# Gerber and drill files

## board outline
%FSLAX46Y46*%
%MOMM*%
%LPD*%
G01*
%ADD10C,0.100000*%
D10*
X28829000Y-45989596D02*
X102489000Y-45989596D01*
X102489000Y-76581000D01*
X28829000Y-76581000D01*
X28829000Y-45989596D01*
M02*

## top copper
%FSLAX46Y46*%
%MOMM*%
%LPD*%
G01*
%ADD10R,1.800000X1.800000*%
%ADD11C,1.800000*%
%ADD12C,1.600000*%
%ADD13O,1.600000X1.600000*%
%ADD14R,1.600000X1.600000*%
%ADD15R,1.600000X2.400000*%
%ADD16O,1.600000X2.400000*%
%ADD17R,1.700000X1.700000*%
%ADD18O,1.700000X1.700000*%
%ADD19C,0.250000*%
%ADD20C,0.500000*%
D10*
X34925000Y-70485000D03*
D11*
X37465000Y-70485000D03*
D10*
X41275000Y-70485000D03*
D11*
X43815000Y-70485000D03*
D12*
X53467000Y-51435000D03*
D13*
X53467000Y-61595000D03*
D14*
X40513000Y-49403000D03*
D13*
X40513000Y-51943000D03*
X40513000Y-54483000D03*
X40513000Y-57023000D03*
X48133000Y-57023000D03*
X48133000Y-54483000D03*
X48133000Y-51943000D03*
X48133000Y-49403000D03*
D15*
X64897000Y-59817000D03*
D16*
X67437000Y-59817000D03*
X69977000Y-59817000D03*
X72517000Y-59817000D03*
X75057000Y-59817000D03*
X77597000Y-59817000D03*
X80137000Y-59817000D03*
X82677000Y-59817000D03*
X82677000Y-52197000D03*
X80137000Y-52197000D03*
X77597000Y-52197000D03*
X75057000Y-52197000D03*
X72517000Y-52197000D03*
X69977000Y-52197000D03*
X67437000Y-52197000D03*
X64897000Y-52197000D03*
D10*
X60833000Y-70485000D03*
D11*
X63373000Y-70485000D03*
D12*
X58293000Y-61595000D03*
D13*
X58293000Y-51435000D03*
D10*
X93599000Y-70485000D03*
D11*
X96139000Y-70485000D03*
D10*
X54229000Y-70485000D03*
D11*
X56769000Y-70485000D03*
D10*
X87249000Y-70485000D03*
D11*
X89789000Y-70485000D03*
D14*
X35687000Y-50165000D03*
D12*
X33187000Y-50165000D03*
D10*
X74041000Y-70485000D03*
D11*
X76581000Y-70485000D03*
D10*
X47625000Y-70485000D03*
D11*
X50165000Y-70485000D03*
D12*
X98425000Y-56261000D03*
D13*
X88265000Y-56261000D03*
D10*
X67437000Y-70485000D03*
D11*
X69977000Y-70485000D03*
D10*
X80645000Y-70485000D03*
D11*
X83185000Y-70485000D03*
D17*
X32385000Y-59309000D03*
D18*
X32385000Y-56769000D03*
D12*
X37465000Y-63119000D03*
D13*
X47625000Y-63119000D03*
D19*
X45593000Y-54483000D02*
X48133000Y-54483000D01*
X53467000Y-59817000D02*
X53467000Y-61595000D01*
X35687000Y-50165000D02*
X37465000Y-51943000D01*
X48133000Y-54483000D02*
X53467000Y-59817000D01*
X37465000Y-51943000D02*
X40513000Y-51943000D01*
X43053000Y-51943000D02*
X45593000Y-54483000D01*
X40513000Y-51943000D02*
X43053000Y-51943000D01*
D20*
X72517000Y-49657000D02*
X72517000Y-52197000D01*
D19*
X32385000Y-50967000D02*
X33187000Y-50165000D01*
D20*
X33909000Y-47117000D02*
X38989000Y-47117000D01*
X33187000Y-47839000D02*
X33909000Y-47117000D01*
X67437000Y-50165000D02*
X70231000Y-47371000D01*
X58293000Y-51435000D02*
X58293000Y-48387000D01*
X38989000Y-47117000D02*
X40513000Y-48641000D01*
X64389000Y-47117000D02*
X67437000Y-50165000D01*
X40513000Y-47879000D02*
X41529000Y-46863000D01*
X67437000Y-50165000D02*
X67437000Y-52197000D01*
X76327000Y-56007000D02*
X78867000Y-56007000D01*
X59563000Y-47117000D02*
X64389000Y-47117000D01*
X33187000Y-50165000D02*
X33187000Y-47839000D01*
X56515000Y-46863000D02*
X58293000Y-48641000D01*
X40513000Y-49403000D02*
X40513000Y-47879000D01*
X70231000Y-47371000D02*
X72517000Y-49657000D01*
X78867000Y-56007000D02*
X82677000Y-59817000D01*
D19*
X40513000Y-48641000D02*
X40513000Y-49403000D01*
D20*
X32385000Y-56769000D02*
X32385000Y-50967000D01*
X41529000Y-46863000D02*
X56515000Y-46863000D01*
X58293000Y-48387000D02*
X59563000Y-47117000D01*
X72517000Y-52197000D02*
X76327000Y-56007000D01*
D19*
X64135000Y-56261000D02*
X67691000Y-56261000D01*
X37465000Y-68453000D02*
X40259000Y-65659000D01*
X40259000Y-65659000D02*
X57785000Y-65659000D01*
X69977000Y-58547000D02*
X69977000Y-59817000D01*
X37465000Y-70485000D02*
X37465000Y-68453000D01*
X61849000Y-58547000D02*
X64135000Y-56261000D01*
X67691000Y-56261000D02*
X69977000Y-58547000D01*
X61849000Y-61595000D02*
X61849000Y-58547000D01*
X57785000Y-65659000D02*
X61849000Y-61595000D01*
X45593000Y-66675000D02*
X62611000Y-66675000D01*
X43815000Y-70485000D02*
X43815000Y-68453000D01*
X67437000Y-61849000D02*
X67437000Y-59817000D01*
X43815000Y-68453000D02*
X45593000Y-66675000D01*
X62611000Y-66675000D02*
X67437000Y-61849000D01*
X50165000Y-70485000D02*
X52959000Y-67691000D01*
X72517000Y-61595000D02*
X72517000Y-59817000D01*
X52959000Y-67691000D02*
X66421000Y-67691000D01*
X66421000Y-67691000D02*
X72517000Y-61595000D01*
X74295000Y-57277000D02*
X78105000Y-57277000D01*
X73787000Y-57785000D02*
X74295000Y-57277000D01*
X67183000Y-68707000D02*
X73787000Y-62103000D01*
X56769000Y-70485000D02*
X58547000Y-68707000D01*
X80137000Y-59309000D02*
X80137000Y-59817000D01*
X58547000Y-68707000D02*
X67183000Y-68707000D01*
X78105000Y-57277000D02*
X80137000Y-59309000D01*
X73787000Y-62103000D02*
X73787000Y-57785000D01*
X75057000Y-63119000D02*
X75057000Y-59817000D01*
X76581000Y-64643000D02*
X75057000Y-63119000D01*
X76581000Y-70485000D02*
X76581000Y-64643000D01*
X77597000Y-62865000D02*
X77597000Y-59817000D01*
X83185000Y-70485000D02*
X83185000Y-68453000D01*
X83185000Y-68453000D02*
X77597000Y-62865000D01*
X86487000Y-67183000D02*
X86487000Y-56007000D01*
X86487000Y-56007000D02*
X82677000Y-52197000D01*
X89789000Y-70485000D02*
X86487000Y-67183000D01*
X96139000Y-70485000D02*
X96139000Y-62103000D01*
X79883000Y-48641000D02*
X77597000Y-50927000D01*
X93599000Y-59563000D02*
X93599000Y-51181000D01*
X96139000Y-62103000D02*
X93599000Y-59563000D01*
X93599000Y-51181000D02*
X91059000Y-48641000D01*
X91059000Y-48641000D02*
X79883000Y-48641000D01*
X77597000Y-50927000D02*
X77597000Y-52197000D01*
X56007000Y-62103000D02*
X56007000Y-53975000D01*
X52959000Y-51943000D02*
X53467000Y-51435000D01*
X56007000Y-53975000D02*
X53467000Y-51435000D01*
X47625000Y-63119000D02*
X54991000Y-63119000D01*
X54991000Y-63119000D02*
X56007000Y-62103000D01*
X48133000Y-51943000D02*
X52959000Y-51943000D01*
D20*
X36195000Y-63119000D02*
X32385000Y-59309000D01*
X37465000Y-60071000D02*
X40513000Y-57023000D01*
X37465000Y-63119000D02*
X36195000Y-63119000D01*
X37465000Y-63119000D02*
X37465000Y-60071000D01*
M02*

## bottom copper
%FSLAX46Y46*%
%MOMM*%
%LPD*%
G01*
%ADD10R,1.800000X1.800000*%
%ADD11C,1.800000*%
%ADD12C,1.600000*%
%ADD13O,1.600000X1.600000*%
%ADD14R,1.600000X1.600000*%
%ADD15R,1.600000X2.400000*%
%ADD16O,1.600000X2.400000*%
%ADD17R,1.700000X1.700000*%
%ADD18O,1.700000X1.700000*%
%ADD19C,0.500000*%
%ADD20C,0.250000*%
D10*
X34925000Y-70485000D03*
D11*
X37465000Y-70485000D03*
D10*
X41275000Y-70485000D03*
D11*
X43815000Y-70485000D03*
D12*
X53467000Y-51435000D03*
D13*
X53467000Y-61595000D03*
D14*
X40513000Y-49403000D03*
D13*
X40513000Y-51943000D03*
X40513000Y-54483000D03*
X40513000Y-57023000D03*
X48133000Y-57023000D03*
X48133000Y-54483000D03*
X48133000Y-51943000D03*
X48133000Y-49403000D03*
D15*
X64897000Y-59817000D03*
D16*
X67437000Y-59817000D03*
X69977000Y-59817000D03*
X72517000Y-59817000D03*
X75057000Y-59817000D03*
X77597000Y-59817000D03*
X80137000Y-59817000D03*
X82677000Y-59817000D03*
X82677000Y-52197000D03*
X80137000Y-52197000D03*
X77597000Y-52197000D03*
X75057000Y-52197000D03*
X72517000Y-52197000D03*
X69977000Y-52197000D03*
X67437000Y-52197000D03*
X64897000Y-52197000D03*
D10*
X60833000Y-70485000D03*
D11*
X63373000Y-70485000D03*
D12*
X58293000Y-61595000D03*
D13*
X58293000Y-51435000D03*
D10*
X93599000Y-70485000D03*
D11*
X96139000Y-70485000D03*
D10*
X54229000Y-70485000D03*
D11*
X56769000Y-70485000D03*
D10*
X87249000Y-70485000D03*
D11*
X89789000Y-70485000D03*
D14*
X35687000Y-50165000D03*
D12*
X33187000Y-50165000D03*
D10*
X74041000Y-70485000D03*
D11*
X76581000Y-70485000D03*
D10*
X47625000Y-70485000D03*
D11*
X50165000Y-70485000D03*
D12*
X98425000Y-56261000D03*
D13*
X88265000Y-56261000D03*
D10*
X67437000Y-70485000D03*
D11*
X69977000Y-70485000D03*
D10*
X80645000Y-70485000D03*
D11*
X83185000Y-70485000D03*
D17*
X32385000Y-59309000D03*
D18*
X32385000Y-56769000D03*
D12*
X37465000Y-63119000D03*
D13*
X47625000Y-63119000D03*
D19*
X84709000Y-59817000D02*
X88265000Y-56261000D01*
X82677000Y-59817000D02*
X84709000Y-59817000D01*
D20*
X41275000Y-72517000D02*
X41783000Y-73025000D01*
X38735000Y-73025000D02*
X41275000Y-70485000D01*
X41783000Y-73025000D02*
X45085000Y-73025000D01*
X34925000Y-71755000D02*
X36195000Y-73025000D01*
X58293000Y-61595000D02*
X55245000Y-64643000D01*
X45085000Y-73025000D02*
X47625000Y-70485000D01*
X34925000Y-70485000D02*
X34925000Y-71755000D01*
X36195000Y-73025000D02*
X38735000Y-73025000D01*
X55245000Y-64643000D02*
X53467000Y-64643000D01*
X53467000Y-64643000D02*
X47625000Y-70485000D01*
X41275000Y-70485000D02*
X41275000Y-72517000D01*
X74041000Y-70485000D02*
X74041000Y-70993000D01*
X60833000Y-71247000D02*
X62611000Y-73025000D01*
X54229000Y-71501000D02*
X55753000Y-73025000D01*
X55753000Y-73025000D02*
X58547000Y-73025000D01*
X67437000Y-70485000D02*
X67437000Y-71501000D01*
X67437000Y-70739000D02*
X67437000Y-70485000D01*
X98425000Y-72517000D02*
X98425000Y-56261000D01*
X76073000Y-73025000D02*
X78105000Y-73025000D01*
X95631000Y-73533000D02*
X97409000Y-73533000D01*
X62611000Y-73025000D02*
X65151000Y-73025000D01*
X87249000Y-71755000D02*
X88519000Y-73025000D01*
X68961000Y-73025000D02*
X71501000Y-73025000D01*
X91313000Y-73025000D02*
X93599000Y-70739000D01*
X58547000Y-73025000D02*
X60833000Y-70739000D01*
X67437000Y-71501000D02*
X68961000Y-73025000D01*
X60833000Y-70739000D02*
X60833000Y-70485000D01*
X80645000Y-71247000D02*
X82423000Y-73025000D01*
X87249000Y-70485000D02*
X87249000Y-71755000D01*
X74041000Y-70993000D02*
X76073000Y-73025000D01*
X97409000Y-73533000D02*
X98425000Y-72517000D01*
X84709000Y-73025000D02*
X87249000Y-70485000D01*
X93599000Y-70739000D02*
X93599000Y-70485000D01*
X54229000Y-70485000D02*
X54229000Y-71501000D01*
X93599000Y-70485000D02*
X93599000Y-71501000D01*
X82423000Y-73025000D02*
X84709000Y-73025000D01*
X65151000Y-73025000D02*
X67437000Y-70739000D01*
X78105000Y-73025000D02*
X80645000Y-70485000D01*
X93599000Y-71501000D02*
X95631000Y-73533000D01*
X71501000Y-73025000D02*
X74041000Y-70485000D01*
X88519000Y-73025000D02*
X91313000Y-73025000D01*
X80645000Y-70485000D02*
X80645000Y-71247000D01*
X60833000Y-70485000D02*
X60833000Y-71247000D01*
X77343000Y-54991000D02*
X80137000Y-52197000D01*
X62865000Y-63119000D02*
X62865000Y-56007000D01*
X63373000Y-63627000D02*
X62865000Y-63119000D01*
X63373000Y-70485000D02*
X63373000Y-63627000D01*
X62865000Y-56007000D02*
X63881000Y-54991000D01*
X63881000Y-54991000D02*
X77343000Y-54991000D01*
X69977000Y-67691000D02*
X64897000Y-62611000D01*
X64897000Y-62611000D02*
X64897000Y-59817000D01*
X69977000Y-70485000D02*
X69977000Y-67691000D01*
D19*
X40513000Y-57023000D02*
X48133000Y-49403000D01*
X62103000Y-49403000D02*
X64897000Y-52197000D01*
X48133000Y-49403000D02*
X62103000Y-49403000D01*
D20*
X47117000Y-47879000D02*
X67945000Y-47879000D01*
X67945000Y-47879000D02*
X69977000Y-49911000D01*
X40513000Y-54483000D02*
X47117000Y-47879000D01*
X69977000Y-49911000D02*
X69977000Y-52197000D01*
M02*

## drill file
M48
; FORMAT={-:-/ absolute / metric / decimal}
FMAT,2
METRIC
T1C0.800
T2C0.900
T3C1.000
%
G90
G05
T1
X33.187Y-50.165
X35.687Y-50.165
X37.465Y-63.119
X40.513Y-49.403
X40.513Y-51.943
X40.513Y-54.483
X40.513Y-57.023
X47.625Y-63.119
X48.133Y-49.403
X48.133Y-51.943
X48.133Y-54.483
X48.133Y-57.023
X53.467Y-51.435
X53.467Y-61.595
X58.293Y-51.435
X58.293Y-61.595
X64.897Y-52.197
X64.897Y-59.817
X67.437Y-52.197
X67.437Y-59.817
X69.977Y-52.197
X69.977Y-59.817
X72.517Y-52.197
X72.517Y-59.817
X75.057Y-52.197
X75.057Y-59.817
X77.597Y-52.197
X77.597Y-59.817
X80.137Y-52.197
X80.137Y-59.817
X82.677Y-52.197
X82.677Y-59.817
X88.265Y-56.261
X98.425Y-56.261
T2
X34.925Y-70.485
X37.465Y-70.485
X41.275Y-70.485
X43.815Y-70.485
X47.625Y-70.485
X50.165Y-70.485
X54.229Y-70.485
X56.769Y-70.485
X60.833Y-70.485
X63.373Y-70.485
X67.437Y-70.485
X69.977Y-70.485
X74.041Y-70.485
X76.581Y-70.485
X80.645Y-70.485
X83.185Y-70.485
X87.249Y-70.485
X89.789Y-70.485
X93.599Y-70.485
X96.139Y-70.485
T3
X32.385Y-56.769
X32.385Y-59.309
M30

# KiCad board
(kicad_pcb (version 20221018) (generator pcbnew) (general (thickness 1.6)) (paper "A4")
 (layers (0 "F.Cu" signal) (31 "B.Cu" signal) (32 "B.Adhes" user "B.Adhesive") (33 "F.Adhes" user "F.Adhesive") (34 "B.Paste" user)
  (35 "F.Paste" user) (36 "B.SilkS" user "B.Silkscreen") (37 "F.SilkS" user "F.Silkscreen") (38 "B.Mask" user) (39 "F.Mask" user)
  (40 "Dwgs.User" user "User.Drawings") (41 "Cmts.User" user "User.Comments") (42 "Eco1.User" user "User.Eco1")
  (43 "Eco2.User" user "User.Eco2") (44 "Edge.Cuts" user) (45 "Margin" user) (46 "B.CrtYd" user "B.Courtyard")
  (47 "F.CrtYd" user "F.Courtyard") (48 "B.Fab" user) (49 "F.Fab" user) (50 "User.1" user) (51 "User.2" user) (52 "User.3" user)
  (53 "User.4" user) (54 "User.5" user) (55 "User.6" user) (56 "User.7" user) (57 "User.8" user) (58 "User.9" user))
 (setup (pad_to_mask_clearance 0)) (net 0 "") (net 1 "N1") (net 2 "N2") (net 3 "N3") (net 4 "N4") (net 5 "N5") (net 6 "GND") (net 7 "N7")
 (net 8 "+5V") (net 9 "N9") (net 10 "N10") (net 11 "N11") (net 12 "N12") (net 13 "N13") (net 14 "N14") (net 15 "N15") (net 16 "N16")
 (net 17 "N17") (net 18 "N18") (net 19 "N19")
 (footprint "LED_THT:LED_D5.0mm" (layer "F.Cu") (at 34.925 70.485)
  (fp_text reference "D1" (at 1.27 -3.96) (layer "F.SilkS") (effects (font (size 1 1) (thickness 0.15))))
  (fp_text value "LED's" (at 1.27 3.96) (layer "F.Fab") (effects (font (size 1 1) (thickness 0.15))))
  (pad "1" thru_hole rect (at 0 0) (size 1.8 1.8) (drill 0.9) (layers "*.Cu" "*.Mask") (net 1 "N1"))
  (pad "2" thru_hole circle (at 2.54 0) (size 1.8 1.8) (drill 0.9) (layers "*.Cu" "*.Mask") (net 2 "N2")))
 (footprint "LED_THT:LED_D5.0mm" (layer "F.Cu") (at 41.275 70.485)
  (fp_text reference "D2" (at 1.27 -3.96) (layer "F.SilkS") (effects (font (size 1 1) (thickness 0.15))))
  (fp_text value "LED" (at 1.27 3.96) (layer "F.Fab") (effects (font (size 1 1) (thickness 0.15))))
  (pad "1" thru_hole rect (at 0 0) (size 1.8 1.8) (drill 0.9) (layers "*.Cu" "*.Mask") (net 1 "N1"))
  (pad "2" thru_hole circle (at 2.54 0) (size 1.8 1.8) (drill 0.9) (layers "*.Cu" "*.Mask") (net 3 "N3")))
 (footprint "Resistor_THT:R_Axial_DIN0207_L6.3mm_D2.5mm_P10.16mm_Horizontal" (layer "F.Cu") (at 53.467 51.435 -90)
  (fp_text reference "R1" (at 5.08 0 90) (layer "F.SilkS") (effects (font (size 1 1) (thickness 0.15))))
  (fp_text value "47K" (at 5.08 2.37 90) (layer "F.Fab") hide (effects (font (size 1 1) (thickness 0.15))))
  (pad "1" thru_hole circle (at 0 0 270) (size 1.6 1.6) (drill 0.8) (layers "*.Cu" "*.Mask") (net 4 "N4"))
  (pad "2" thru_hole oval (at 10.16 0 270) (size 1.6 1.6) (drill 0.8) (layers "*.Cu" "*.Mask") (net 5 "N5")))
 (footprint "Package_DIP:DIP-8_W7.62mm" (layer "F.Cu") (at 40.513 49.403)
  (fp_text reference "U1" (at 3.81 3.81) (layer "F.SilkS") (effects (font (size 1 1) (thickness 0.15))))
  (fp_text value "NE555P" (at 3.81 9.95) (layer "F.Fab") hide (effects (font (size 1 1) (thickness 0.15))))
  (pad "1" thru_hole rect (at 0 0) (size 1.6 1.6) (drill 0.8) (layers "*.Cu" "*.Mask") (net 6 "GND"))
  (pad "2" thru_hole oval (at 0 2.54) (size 1.6 1.6) (drill 0.8) (layers "*.Cu" "*.Mask") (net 5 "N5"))
  (pad "3" thru_hole oval (at 0 5.08) (size 1.6 1.6) (drill 0.8) (layers "*.Cu" "*.Mask") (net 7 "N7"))
  (pad "4" thru_hole oval (at 0 7.62) (size 1.6 1.6) (drill 0.8) (layers "*.Cu" "*.Mask") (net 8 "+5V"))
  (pad "5" thru_hole oval (at 7.62 7.62) (size 1.6 1.6) (drill 0.8) (layers "*.Cu" "*.Mask") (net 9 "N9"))
  (pad "6" thru_hole oval (at 7.62 5.08) (size 1.6 1.6) (drill 0.8) (layers "*.Cu" "*.Mask") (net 5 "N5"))
  (pad "7" thru_hole oval (at 7.62 2.54) (size 1.6 1.6) (drill 0.8) (layers "*.Cu" "*.Mask") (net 4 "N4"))
  (pad "8" thru_hole oval (at 7.62 0) (size 1.6 1.6) (drill 0.8) (layers "*.Cu" "*.Mask") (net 8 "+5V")))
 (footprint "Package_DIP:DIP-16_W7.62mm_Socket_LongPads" (layer "F.Cu") (at 64.897 59.817 90)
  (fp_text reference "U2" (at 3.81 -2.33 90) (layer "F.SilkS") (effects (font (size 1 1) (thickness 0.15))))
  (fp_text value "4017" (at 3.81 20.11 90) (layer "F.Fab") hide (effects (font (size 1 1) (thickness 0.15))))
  (pad "1" thru_hole rect (at 0 0 90) (size 2.4 1.6) (drill 0.8) (layers "*.Cu" "*.Mask") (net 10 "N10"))
  (pad "2" thru_hole oval (at 0 2.54 90) (size 2.4 1.6) (drill 0.8) (layers "*.Cu" "*.Mask") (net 3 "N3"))
  (pad "3" thru_hole oval (at 0 5.08 90) (size 2.4 1.6) (drill 0.8) (layers "*.Cu" "*.Mask") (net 2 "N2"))
  (pad "4" thru_hole oval (at 0 7.62 90) (size 2.4 1.6) (drill 0.8) (layers "*.Cu" "*.Mask") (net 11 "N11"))
  (pad "5" thru_hole oval (at 0 10.16 90) (size 2.4 1.6) (drill 0.8) (layers "*.Cu" "*.Mask") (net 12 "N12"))
  (pad "6" thru_hole oval (at 0 12.7 90) (size 2.4 1.6) (drill 0.8) (layers "*.Cu" "*.Mask") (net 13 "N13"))
  (pad "7" thru_hole oval (at 0 15.24 90) (size 2.4 1.6) (drill 0.8) (layers "*.Cu" "*.Mask") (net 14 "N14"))
  (pad "8" thru_hole oval (at 0 17.78 90) (size 2.4 1.6) (drill 0.8) (layers "*.Cu" "*.Mask") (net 6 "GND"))
  (pad "9" thru_hole oval (at 7.62 17.78 90) (size 2.4 1.6) (drill 0.8) (layers "*.Cu" "*.Mask") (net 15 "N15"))
  (pad "10" thru_hole oval (at 7.62 15.24 90) (size 2.4 1.6) (drill 0.8) (layers "*.Cu" "*.Mask") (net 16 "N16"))
  (pad "11" thru_hole oval (at 7.62 12.7 90) (size 2.4 1.6) (drill 0.8) (layers "*.Cu" "*.Mask") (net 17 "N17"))
  (pad "12" thru_hole oval (at 7.62 10.16 90) (size 2.4 1.6) (drill 0.8) (layers "*.Cu" "*.Mask") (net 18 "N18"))
  (pad "13" thru_hole oval (at 7.62 7.62 90) (size 2.4 1.6) (drill 0.8) (layers "*.Cu" "*.Mask") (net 6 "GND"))
  (pad "14" thru_hole oval (at 7.62 5.08 90) (size 2.4 1.6) (drill 0.8) (layers "*.Cu" "*.Mask") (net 7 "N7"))
  (pad "15" thru_hole oval (at 7.62 2.54 90) (size 2.4 1.6) (drill 0.8) (layers "*.Cu" "*.Mask") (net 6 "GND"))
  (pad "16" thru_hole oval (at 7.62 0 90) (size 2.4 1.6) (drill 0.8) (layers "*.Cu" "*.Mask") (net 8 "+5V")))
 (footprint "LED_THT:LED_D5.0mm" (layer "F.Cu") (at 60.833 70.485)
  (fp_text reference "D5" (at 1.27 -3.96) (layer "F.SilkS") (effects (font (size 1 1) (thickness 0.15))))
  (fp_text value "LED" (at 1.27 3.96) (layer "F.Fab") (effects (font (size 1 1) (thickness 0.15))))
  (pad "1" thru_hole rect (at 0 0) (size 1.8 1.8) (drill 0.9) (layers "*.Cu" "*.Mask") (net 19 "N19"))
  (pad "2" thru_hole circle (at 2.54 0) (size 1.8 1.8) (drill 0.9) (layers "*.Cu" "*.Mask") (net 16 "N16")))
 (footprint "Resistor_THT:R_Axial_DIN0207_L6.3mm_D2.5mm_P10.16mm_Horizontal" (layer "F.Cu") (at 58.293 61.595 90)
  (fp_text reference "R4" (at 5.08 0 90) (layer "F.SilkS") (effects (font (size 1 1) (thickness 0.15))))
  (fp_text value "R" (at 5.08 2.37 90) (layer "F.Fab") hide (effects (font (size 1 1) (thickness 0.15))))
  (pad "1" thru_hole circle (at 0 0 90) (size 1.6 1.6) (drill 0.8) (layers "*.Cu" "*.Mask") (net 1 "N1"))
  (pad "2" thru_hole oval (at 10.16 0 90) (size 1.6 1.6) (drill 0.8) (layers "*.Cu" "*.Mask") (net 6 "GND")))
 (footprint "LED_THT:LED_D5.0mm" (layer "F.Cu") (at 93.599 70.485)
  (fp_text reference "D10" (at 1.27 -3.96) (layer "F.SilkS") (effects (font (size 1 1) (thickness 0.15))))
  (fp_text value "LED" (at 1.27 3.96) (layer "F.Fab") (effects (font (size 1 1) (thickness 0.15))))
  (pad "1" thru_hole rect (at 0 0) (size 1.8 1.8) (drill 0.9) (layers "*.Cu" "*.Mask") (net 19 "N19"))
  (pad "2" thru_hole circle (at 2.54 0) (size 1.8 1.8) (drill 0.9) (layers "*.Cu" "*.Mask") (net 17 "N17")))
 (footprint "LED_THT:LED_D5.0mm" (layer "F.Cu") (at 54.229 70.485)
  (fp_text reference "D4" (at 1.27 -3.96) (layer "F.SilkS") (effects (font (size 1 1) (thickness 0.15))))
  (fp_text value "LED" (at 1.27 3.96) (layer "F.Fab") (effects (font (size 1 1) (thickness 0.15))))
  (pad "1" thru_hole rect (at 0 0) (size 1.8 1.8) (drill 0.9) (layers "*.Cu" "*.Mask") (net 19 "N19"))
  (pad "2" thru_hole circle (at 2.54 0) (size 1.8 1.8) (drill 0.9) (layers "*.Cu" "*.Mask") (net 14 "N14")))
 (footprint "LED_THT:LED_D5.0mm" (layer "F.Cu") (at 87.249 70.485)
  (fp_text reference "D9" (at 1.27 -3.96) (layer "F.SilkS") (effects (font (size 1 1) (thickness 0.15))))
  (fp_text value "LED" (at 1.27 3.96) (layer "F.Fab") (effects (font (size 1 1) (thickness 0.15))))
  (pad "1" thru_hole rect (at 0 0) (size 1.8 1.8) (drill 0.9) (layers "*.Cu" "*.Mask") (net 19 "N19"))
  (pad "2" thru_hole circle (at 2.54 0) (size 1.8 1.8) (drill 0.9) (layers "*.Cu" "*.Mask") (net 15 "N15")))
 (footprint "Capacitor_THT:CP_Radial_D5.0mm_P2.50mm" (layer "F.Cu") (at 35.687 50.165 180)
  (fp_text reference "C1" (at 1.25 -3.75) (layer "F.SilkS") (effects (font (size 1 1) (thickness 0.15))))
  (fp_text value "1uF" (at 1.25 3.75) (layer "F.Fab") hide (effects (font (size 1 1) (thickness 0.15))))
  (pad "1" thru_hole rect (at 0 0 180) (size 1.6 1.6) (drill 0.8) (layers "*.Cu" "*.Mask") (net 5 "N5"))
  (pad "2" thru_hole circle (at 2.5 0 180) (size 1.6 1.6) (drill 0.8) (layers "*.Cu" "*.Mask") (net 6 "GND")))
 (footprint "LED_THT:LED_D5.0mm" (layer "F.Cu") (at 74.041 70.485)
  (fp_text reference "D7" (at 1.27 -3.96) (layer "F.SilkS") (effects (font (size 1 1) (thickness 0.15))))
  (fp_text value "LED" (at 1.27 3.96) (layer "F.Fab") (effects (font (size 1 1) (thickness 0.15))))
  (pad "1" thru_hole rect (at 0 0) (size 1.8 1.8) (drill 0.9) (layers "*.Cu" "*.Mask") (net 19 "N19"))
  (pad "2" thru_hole circle (at 2.54 0) (size 1.8 1.8) (drill 0.9) (layers "*.Cu" "*.Mask") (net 12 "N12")))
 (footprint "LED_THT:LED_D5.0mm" (layer "F.Cu") (at 47.625 70.485)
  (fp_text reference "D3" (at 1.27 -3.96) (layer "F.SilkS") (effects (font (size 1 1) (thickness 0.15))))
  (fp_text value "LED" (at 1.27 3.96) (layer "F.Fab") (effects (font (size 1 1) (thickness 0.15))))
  (pad "1" thru_hole rect (at 0 0) (size 1.8 1.8) (drill 0.9) (layers "*.Cu" "*.Mask") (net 1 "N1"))
  (pad "2" thru_hole circle (at 2.54 0) (size 1.8 1.8) (drill 0.9) (layers "*.Cu" "*.Mask") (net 11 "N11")))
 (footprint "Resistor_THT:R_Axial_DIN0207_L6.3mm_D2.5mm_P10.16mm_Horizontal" (layer "F.Cu") (at 98.425 56.261 180)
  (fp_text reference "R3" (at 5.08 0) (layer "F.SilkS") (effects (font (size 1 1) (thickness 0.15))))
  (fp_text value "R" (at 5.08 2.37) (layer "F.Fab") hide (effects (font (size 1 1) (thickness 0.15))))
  (pad "1" thru_hole circle (at 0 0 180) (size 1.6 1.6) (drill 0.8) (layers "*.Cu" "*.Mask") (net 19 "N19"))
  (pad "2" thru_hole oval (at 10.16 0 180) (size 1.6 1.6) (drill 0.8) (layers "*.Cu" "*.Mask") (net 6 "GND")))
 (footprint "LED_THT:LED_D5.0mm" (layer "F.Cu") (at 67.437 70.485)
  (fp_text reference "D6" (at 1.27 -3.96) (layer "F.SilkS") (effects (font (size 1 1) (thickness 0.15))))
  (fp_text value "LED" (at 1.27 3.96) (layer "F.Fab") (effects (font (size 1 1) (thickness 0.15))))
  (pad "1" thru_hole rect (at 0 0) (size 1.8 1.8) (drill 0.9) (layers "*.Cu" "*.Mask") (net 19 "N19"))
  (pad "2" thru_hole circle (at 2.54 0) (size 1.8 1.8) (drill 0.9) (layers "*.Cu" "*.Mask") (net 10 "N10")))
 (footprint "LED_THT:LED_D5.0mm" (layer "F.Cu") (at 80.645 70.485)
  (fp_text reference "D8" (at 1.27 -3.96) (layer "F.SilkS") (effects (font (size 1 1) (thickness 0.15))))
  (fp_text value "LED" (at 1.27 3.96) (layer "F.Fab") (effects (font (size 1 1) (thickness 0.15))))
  (pad "1" thru_hole rect (at 0 0) (size 1.8 1.8) (drill 0.9) (layers "*.Cu" "*.Mask") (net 19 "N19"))
  (pad "2" thru_hole circle (at 2.54 0) (size 1.8 1.8) (drill 0.9) (layers "*.Cu" "*.Mask") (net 13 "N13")))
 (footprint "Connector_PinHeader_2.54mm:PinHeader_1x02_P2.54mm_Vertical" (layer "F.Cu") (at 32.385 59.309 180)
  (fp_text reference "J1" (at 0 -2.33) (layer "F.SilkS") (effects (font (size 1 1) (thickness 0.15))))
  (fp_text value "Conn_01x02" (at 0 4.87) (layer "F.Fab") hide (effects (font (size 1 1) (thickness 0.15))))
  (pad "1" thru_hole rect (at 0 0 180) (size 1.7 1.7) (drill 1) (layers "*.Cu" "*.Mask") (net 8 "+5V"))
  (pad "2" thru_hole oval (at 0 2.54 180) (size 1.7 1.7) (drill 1) (layers "*.Cu" "*.Mask") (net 6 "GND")))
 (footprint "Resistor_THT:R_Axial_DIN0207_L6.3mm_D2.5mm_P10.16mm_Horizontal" (layer "F.Cu") (at 37.465 63.119)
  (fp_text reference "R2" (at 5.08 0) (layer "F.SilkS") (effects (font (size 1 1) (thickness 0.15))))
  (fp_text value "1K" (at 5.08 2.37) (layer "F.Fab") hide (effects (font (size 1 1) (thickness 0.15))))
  (pad "1" thru_hole circle (at 0 0) (size 1.6 1.6) (drill 0.8) (layers "*.Cu" "*.Mask") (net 8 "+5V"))
  (pad "2" thru_hole oval (at 10.16 0) (size 1.6 1.6) (drill 0.8) (layers "*.Cu" "*.Mask") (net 4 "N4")))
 (gr_rect (start 28.829 45.989596) (end 102.489 76.581) (stroke (width 0.1) (type default)) (fill none) (layer "Edge.Cuts"))
 (segment (start 45.593 54.483) (end 48.133 54.483) (width 0.25) (layer "F.Cu") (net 5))
 (segment (start 53.467 59.817) (end 53.467 61.595) (width 0.25) (layer "F.Cu") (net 5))
 (segment (start 35.687 50.165) (end 37.465 51.943) (width 0.25) (layer "F.Cu") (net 5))
 (segment (start 48.133 54.483) (end 53.467 59.817) (width 0.25) (layer "F.Cu") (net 5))
 (segment (start 37.465 51.943) (end 40.513 51.943) (width 0.25) (layer "F.Cu") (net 5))
 (segment (start 43.053 51.943) (end 45.593 54.483) (width 0.25) (layer "F.Cu") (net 5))
 (segment (start 40.513 51.943) (end 43.053 51.943) (width 0.25) (layer "F.Cu") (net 5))
 (segment (start 72.517 49.657) (end 72.517 52.197) (width 0.5) (layer "F.Cu") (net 6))
 (segment (start 32.385 50.967) (end 33.187 50.165) (width 0.25) (layer "F.Cu") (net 6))
 (segment (start 33.909 47.117) (end 38.989 47.117) (width 0.5) (layer "F.Cu") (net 6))
 (segment (start 33.187 47.839) (end 33.909 47.117) (width 0.5) (layer "F.Cu") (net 6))
 (segment (start 67.437 50.165) (end 70.231 47.371) (width 0.5) (layer "F.Cu") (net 6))
 (segment (start 58.293 51.435) (end 58.293 48.387) (width 0.5) (layer "F.Cu") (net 6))
 (segment (start 38.989 47.117) (end 40.513 48.641) (width 0.5) (layer "F.Cu") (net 6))
 (segment (start 64.389 47.117) (end 67.437 50.165) (width 0.5) (layer "F.Cu") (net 6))
 (segment (start 40.513 47.879) (end 41.529 46.863) (width 0.5) (layer "F.Cu") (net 6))
 (segment (start 67.437 50.165) (end 67.437 52.197) (width 0.5) (layer "F.Cu") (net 6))
 (segment (start 76.327 56.007) (end 78.867 56.007) (width 0.5) (layer "F.Cu") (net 6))
 (segment (start 59.563 47.117) (end 64.389 47.117) (width 0.5) (layer "F.Cu") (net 6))
 (segment (start 33.187 50.165) (end 33.187 47.839) (width 0.5) (layer "F.Cu") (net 6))
 (segment (start 56.515 46.863) (end 58.293 48.641) (width 0.5) (layer "F.Cu") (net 6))
 (segment (start 40.513 49.403) (end 40.513 47.879) (width 0.5) (layer "F.Cu") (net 6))
 (segment (start 70.231 47.371) (end 72.517 49.657) (width 0.5) (layer "F.Cu") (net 6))
 (segment (start 78.867 56.007) (end 82.677 59.817) (width 0.5) (layer "F.Cu") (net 6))
 (segment (start 40.513 48.641) (end 40.513 49.403) (width 0.25) (layer "F.Cu") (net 6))
 (segment (start 32.385 56.769) (end 32.385 50.967) (width 0.5) (layer "F.Cu") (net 6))
 (segment (start 41.529 46.863) (end 56.515 46.863) (width 0.5) (layer "F.Cu") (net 6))
 (segment (start 58.293 48.387) (end 59.563 47.117) (width 0.5) (layer "F.Cu") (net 6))
 (segment (start 72.517 52.197) (end 76.327 56.007) (width 0.5) (layer "F.Cu") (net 6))
 (segment (start 84.709 59.817) (end 88.265 56.261) (width 0.5) (layer "B.Cu") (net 6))
 (segment (start 82.677 59.817) (end 84.709 59.817) (width 0.5) (layer "B.Cu") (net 6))
 (segment (start 41.275 72.517) (end 41.783 73.025) (width 0.25) (layer "B.Cu") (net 1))
 (segment (start 38.735 73.025) (end 41.275 70.485) (width 0.25) (layer "B.Cu") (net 1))
 (segment (start 41.783 73.025) (end 45.085 73.025) (width 0.25) (layer "B.Cu") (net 1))
 (segment (start 34.925 71.755) (end 36.195 73.025) (width 0.25) (layer "B.Cu") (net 1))
 (segment (start 58.293 61.595) (end 55.245 64.643) (width 0.25) (layer "B.Cu") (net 1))
 (segment (start 45.085 73.025) (end 47.625 70.485) (width 0.25) (layer "B.Cu") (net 1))
 (segment (start 34.925 70.485) (end 34.925 71.755) (width 0.25) (layer "B.Cu") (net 1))
 (segment (start 36.195 73.025) (end 38.735 73.025) (width 0.25) (layer "B.Cu") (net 1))
 (segment (start 55.245 64.643) (end 53.467 64.643) (width 0.25) (layer "B.Cu") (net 1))
 (segment (start 53.467 64.643) (end 47.625 70.485) (width 0.25) (layer "B.Cu") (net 1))
 (segment (start 41.275 70.485) (end 41.275 72.517) (width 0.25) (layer "B.Cu") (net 1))
 (segment (start 64.135 56.261) (end 67.691 56.261) (width 0.25) (layer "F.Cu") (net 2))
 (segment (start 37.465 68.453) (end 40.259 65.659) (width 0.25) (layer "F.Cu") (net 2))
 (segment (start 40.259 65.659) (end 57.785 65.659) (width 0.25) (layer "F.Cu") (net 2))
 (segment (start 69.977 58.547) (end 69.977 59.817) (width 0.25) (layer "F.Cu") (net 2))
 (segment (start 37.465 70.485) (end 37.465 68.453) (width 0.25) (layer "F.Cu") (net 2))
 (segment (start 61.849 58.547) (end 64.135 56.261) (width 0.25) (layer "F.Cu") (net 2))
 (segment (start 67.691 56.261) (end 69.977 58.547) (width 0.25) (layer "F.Cu") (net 2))
 (segment (start 61.849 61.595) (end 61.849 58.547) (width 0.25) (layer "F.Cu") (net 2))
 (segment (start 57.785 65.659) (end 61.849 61.595) (width 0.25) (layer "F.Cu") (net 2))
 (segment (start 45.593 66.675) (end 62.611 66.675) (width 0.25) (layer "F.Cu") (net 3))
 (segment (start 43.815 70.485) (end 43.815 68.453) (width 0.25) (layer "F.Cu") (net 3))
 (segment (start 67.437 61.849) (end 67.437 59.817) (width 0.25) (layer "F.Cu") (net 3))
 (segment (start 43.815 68.453) (end 45.593 66.675) (width 0.25) (layer "F.Cu") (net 3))
 (segment (start 62.611 66.675) (end 67.437 61.849) (width 0.25) (layer "F.Cu") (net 3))
 (segment (start 50.165 70.485) (end 52.959 67.691) (width 0.25) (layer "F.Cu") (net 11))
 (segment (start 72.517 61.595) (end 72.517 59.817) (width 0.25) (layer "F.Cu") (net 11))
 (segment (start 52.959 67.691) (end 66.421 67.691) (width 0.25) (layer "F.Cu") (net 11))
 (segment (start 66.421 67.691) (end 72.517 61.595) (width 0.25) (layer "F.Cu") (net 11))
 (segment (start 74.041 70.485) (end 74.041 70.993) (width 0.25) (layer "B.Cu") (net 19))
 (segment (start 60.833 71.247) (end 62.611 73.025) (width 0.25) (layer "B.Cu") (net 19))
 (segment (start 54.229 71.501) (end 55.753 73.025) (width 0.25) (layer "B.Cu") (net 19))
 (segment (start 55.753 73.025) (end 58.547 73.025) (width 0.25) (layer "B.Cu") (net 19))
 (segment (start 67.437 70.485) (end 67.437 71.501) (width 0.25) (layer "B.Cu") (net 19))
 (segment (start 67.437 70.739) (end 67.437 70.485) (width 0.25) (layer "B.Cu") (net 19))
 (segment (start 98.425 72.517) (end 98.425 56.261) (width 0.25) (layer "B.Cu") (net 19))
 (segment (start 76.073 73.025) (end 78.105 73.025) (width 0.25) (layer "B.Cu") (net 19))
 (segment (start 95.631 73.533) (end 97.409 73.533) (width 0.25) (layer "B.Cu") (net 19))
 (segment (start 62.611 73.025) (end 65.151 73.025) (width 0.25) (layer "B.Cu") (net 19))
 (segment (start 87.249 71.755) (end 88.519 73.025) (width 0.25) (layer "B.Cu") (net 19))
 (segment (start 68.961 73.025) (end 71.501 73.025) (width 0.25) (layer "B.Cu") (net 19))
 (segment (start 91.313 73.025) (end 93.599 70.739) (width 0.25) (layer "B.Cu") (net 19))
 (segment (start 58.547 73.025) (end 60.833 70.739) (width 0.25) (layer "B.Cu") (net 19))
 (segment (start 67.437 71.501) (end 68.961 73.025) (width 0.25) (layer "B.Cu") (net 19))
 (segment (start 60.833 70.739) (end 60.833 70.485) (width 0.25) (layer "B.Cu") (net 19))
 (segment (start 80.645 71.247) (end 82.423 73.025) (width 0.25) (layer "B.Cu") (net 19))
 (segment (start 87.249 70.485) (end 87.249 71.755) (width 0.25) (layer "B.Cu") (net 19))
 (segment (start 74.041 70.993) (end 76.073 73.025) (width 0.25) (layer "B.Cu") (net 19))
 (segment (start 97.409 73.533) (end 98.425 72.517) (width 0.25) (layer "B.Cu") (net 19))
 (segment (start 84.709 73.025) (end 87.249 70.485) (width 0.25) (layer "B.Cu") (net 19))
 (segment (start 93.599 70.739) (end 93.599 70.485) (width 0.25) (layer "B.Cu") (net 19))
 (segment (start 54.229 70.485) (end 54.229 71.501) (width 0.25) (layer "B.Cu") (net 19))
 (segment (start 93.599 70.485) (end 93.599 71.501) (width 0.25) (layer "B.Cu") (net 19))
 (segment (start 82.423 73.025) (end 84.709 73.025) (width 0.25) (layer "B.Cu") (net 19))
 (segment (start 65.151 73.025) (end 67.437 70.739) (width 0.25) (layer "B.Cu") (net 19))
 (segment (start 78.105 73.025) (end 80.645 70.485) (width 0.25) (layer "B.Cu") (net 19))
 (segment (start 93.599 71.501) (end 95.631 73.533) (width 0.25) (layer "B.Cu") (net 19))
 (segment (start 71.501 73.025) (end 74.041 70.485) (width 0.25) (layer "B.Cu") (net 19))
 (segment (start 88.519 73.025) (end 91.313 73.025) (width 0.25) (layer "B.Cu") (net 19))
 (segment (start 80.645 70.485) (end 80.645 71.247) (width 0.25) (layer "B.Cu") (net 19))
 (segment (start 60.833 70.485) (end 60.833 71.247) (width 0.25) (layer "B.Cu") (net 19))
 (segment (start 74.295 57.277) (end 78.105 57.277) (width 0.25) (layer "F.Cu") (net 14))
 (segment (start 73.787 57.785) (end 74.295 57.277) (width 0.25) (layer "F.Cu") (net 14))
 (segment (start 67.183 68.707) (end 73.787 62.103) (width 0.25) (layer "F.Cu") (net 14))
 (segment (start 56.769 70.485) (end 58.547 68.707) (width 0.25) (layer "F.Cu") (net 14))
 (segment (start 80.137 59.309) (end 80.137 59.817) (width 0.25) (layer "F.Cu") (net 14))
 (segment (start 58.547 68.707) (end 67.183 68.707) (width 0.25) (layer "F.Cu") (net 14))
 (segment (start 78.105 57.277) (end 80.137 59.309) (width 0.25) (layer "F.Cu") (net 14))
 (segment (start 73.787 62.103) (end 73.787 57.785) (width 0.25) (layer "F.Cu") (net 14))
 (segment (start 77.343 54.991) (end 80.137 52.197) (width 0.25) (layer "B.Cu") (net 16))
 (segment (start 62.865 63.119) (end 62.865 56.007) (width 0.25) (layer "B.Cu") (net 16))
 (segment (start 63.373 63.627) (end 62.865 63.119) (width 0.25) (layer "B.Cu") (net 16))
 (segment (start 63.373 70.485) (end 63.373 63.627) (width 0.25) (layer "B.Cu") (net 16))
 (segment (start 62.865 56.007) (end 63.881 54.991) (width 0.25) (layer "B.Cu") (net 16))
 (segment (start 63.881 54.991) (end 77.343 54.991) (width 0.25) (layer "B.Cu") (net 16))
 (segment (start 69.977 67.691) (end 64.897 62.611) (width 0.25) (layer "B.Cu") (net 10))
 (segment (start 64.897 62.611) (end 64.897 59.817) (width 0.25) (layer "B.Cu") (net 10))
 (segment (start 69.977 70.485) (end 69.977 67.691) (width 0.25) (layer "B.Cu") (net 10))
 (segment (start 75.057 63.119) (end 75.057 59.817) (width 0.25) (layer "F.Cu") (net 12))
 (segment (start 76.581 64.643) (end 75.057 63.119) (width 0.25) (layer "F.Cu") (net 12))
 (segment (start 76.581 70.485) (end 76.581 64.643) (width 0.25) (layer "F.Cu") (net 12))
 (segment (start 77.597 62.865) (end 77.597 59.817) (width 0.25) (layer "F.Cu") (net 13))
 (segment (start 83.185 70.485) (end 83.185 68.453) (width 0.25) (layer "F.Cu") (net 13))
 (segment (start 83.185 68.453) (end 77.597 62.865) (width 0.25) (layer "F.Cu") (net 13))
 (segment (start 86.487 67.183) (end 86.487 56.007) (width 0.25) (layer "F.Cu") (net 15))
 (segment (start 86.487 56.007) (end 82.677 52.197) (width 0.25) (layer "F.Cu") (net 15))
 (segment (start 89.789 70.485) (end 86.487 67.183) (width 0.25) (layer "F.Cu") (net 15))
 (segment (start 96.139 70.485) (end 96.139 62.103) (width 0.25) (layer "F.Cu") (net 17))
 (segment (start 79.883 48.641) (end 77.597 50.927) (width 0.25) (layer "F.Cu") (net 17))
 (segment (start 93.599 59.563) (end 93.599 51.181) (width 0.25) (layer "F.Cu") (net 17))
 (segment (start 96.139 62.103) (end 93.599 59.563) (width 0.25) (layer "F.Cu") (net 17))
 (segment (start 93.599 51.181) (end 91.059 48.641) (width 0.25) (layer "F.Cu") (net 17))
 (segment (start 91.059 48.641) (end 79.883 48.641) (width 0.25) (layer "F.Cu") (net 17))
 (segment (start 77.597 50.927) (end 77.597 52.197) (width 0.25) (layer "F.Cu") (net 17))
 (segment (start 56.007 62.103) (end 56.007 53.975) (width 0.25) (layer "F.Cu") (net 4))
 (segment (start 52.959 51.943) (end 53.467 51.435) (width 0.25) (layer "F.Cu") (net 4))
 (segment (start 56.007 53.975) (end 53.467 51.435) (width 0.25) (layer "F.Cu") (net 4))
 (segment (start 47.625 63.119) (end 54.991 63.119) (width 0.25) (layer "F.Cu") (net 4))
 (segment (start 54.991 63.119) (end 56.007 62.103) (width 0.25) (layer "F.Cu") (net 4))
 (segment (start 48.133 51.943) (end 52.959 51.943) (width 0.25) (layer "F.Cu") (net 4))
 (segment (start 36.195 63.119) (end 32.385 59.309) (width 0.5) (layer "F.Cu") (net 8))
 (segment (start 37.465 60.071) (end 40.513 57.023) (width 0.5) (layer "F.Cu") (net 8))
 (segment (start 37.465 63.119) (end 36.195 63.119) (width 0.5) (layer "F.Cu") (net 8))
 (segment (start 37.465 63.119) (end 37.465 60.071) (width 0.5) (layer "F.Cu") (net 8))
 (segment (start 40.513 57.023) (end 48.133 49.403) (width 0.5) (layer "B.Cu") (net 8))
 (segment (start 62.103 49.403) (end 64.897 52.197) (width 0.5) (layer "B.Cu") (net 8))
 (segment (start 48.133 49.403) (end 62.103 49.403) (width 0.5) (layer "B.Cu") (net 8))
 (segment (start 47.117 47.879) (end 67.945 47.879) (width 0.25) (layer "B.Cu") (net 7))
 (segment (start 67.945 47.879) (end 69.977 49.911) (width 0.25) (layer "B.Cu") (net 7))
 (segment (start 40.513 54.483) (end 47.117 47.879) (width 0.25) (layer "B.Cu") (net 7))
 (segment (start 69.977 49.911) (end 69.977 52.197) (width 0.25) (layer "B.Cu") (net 7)))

